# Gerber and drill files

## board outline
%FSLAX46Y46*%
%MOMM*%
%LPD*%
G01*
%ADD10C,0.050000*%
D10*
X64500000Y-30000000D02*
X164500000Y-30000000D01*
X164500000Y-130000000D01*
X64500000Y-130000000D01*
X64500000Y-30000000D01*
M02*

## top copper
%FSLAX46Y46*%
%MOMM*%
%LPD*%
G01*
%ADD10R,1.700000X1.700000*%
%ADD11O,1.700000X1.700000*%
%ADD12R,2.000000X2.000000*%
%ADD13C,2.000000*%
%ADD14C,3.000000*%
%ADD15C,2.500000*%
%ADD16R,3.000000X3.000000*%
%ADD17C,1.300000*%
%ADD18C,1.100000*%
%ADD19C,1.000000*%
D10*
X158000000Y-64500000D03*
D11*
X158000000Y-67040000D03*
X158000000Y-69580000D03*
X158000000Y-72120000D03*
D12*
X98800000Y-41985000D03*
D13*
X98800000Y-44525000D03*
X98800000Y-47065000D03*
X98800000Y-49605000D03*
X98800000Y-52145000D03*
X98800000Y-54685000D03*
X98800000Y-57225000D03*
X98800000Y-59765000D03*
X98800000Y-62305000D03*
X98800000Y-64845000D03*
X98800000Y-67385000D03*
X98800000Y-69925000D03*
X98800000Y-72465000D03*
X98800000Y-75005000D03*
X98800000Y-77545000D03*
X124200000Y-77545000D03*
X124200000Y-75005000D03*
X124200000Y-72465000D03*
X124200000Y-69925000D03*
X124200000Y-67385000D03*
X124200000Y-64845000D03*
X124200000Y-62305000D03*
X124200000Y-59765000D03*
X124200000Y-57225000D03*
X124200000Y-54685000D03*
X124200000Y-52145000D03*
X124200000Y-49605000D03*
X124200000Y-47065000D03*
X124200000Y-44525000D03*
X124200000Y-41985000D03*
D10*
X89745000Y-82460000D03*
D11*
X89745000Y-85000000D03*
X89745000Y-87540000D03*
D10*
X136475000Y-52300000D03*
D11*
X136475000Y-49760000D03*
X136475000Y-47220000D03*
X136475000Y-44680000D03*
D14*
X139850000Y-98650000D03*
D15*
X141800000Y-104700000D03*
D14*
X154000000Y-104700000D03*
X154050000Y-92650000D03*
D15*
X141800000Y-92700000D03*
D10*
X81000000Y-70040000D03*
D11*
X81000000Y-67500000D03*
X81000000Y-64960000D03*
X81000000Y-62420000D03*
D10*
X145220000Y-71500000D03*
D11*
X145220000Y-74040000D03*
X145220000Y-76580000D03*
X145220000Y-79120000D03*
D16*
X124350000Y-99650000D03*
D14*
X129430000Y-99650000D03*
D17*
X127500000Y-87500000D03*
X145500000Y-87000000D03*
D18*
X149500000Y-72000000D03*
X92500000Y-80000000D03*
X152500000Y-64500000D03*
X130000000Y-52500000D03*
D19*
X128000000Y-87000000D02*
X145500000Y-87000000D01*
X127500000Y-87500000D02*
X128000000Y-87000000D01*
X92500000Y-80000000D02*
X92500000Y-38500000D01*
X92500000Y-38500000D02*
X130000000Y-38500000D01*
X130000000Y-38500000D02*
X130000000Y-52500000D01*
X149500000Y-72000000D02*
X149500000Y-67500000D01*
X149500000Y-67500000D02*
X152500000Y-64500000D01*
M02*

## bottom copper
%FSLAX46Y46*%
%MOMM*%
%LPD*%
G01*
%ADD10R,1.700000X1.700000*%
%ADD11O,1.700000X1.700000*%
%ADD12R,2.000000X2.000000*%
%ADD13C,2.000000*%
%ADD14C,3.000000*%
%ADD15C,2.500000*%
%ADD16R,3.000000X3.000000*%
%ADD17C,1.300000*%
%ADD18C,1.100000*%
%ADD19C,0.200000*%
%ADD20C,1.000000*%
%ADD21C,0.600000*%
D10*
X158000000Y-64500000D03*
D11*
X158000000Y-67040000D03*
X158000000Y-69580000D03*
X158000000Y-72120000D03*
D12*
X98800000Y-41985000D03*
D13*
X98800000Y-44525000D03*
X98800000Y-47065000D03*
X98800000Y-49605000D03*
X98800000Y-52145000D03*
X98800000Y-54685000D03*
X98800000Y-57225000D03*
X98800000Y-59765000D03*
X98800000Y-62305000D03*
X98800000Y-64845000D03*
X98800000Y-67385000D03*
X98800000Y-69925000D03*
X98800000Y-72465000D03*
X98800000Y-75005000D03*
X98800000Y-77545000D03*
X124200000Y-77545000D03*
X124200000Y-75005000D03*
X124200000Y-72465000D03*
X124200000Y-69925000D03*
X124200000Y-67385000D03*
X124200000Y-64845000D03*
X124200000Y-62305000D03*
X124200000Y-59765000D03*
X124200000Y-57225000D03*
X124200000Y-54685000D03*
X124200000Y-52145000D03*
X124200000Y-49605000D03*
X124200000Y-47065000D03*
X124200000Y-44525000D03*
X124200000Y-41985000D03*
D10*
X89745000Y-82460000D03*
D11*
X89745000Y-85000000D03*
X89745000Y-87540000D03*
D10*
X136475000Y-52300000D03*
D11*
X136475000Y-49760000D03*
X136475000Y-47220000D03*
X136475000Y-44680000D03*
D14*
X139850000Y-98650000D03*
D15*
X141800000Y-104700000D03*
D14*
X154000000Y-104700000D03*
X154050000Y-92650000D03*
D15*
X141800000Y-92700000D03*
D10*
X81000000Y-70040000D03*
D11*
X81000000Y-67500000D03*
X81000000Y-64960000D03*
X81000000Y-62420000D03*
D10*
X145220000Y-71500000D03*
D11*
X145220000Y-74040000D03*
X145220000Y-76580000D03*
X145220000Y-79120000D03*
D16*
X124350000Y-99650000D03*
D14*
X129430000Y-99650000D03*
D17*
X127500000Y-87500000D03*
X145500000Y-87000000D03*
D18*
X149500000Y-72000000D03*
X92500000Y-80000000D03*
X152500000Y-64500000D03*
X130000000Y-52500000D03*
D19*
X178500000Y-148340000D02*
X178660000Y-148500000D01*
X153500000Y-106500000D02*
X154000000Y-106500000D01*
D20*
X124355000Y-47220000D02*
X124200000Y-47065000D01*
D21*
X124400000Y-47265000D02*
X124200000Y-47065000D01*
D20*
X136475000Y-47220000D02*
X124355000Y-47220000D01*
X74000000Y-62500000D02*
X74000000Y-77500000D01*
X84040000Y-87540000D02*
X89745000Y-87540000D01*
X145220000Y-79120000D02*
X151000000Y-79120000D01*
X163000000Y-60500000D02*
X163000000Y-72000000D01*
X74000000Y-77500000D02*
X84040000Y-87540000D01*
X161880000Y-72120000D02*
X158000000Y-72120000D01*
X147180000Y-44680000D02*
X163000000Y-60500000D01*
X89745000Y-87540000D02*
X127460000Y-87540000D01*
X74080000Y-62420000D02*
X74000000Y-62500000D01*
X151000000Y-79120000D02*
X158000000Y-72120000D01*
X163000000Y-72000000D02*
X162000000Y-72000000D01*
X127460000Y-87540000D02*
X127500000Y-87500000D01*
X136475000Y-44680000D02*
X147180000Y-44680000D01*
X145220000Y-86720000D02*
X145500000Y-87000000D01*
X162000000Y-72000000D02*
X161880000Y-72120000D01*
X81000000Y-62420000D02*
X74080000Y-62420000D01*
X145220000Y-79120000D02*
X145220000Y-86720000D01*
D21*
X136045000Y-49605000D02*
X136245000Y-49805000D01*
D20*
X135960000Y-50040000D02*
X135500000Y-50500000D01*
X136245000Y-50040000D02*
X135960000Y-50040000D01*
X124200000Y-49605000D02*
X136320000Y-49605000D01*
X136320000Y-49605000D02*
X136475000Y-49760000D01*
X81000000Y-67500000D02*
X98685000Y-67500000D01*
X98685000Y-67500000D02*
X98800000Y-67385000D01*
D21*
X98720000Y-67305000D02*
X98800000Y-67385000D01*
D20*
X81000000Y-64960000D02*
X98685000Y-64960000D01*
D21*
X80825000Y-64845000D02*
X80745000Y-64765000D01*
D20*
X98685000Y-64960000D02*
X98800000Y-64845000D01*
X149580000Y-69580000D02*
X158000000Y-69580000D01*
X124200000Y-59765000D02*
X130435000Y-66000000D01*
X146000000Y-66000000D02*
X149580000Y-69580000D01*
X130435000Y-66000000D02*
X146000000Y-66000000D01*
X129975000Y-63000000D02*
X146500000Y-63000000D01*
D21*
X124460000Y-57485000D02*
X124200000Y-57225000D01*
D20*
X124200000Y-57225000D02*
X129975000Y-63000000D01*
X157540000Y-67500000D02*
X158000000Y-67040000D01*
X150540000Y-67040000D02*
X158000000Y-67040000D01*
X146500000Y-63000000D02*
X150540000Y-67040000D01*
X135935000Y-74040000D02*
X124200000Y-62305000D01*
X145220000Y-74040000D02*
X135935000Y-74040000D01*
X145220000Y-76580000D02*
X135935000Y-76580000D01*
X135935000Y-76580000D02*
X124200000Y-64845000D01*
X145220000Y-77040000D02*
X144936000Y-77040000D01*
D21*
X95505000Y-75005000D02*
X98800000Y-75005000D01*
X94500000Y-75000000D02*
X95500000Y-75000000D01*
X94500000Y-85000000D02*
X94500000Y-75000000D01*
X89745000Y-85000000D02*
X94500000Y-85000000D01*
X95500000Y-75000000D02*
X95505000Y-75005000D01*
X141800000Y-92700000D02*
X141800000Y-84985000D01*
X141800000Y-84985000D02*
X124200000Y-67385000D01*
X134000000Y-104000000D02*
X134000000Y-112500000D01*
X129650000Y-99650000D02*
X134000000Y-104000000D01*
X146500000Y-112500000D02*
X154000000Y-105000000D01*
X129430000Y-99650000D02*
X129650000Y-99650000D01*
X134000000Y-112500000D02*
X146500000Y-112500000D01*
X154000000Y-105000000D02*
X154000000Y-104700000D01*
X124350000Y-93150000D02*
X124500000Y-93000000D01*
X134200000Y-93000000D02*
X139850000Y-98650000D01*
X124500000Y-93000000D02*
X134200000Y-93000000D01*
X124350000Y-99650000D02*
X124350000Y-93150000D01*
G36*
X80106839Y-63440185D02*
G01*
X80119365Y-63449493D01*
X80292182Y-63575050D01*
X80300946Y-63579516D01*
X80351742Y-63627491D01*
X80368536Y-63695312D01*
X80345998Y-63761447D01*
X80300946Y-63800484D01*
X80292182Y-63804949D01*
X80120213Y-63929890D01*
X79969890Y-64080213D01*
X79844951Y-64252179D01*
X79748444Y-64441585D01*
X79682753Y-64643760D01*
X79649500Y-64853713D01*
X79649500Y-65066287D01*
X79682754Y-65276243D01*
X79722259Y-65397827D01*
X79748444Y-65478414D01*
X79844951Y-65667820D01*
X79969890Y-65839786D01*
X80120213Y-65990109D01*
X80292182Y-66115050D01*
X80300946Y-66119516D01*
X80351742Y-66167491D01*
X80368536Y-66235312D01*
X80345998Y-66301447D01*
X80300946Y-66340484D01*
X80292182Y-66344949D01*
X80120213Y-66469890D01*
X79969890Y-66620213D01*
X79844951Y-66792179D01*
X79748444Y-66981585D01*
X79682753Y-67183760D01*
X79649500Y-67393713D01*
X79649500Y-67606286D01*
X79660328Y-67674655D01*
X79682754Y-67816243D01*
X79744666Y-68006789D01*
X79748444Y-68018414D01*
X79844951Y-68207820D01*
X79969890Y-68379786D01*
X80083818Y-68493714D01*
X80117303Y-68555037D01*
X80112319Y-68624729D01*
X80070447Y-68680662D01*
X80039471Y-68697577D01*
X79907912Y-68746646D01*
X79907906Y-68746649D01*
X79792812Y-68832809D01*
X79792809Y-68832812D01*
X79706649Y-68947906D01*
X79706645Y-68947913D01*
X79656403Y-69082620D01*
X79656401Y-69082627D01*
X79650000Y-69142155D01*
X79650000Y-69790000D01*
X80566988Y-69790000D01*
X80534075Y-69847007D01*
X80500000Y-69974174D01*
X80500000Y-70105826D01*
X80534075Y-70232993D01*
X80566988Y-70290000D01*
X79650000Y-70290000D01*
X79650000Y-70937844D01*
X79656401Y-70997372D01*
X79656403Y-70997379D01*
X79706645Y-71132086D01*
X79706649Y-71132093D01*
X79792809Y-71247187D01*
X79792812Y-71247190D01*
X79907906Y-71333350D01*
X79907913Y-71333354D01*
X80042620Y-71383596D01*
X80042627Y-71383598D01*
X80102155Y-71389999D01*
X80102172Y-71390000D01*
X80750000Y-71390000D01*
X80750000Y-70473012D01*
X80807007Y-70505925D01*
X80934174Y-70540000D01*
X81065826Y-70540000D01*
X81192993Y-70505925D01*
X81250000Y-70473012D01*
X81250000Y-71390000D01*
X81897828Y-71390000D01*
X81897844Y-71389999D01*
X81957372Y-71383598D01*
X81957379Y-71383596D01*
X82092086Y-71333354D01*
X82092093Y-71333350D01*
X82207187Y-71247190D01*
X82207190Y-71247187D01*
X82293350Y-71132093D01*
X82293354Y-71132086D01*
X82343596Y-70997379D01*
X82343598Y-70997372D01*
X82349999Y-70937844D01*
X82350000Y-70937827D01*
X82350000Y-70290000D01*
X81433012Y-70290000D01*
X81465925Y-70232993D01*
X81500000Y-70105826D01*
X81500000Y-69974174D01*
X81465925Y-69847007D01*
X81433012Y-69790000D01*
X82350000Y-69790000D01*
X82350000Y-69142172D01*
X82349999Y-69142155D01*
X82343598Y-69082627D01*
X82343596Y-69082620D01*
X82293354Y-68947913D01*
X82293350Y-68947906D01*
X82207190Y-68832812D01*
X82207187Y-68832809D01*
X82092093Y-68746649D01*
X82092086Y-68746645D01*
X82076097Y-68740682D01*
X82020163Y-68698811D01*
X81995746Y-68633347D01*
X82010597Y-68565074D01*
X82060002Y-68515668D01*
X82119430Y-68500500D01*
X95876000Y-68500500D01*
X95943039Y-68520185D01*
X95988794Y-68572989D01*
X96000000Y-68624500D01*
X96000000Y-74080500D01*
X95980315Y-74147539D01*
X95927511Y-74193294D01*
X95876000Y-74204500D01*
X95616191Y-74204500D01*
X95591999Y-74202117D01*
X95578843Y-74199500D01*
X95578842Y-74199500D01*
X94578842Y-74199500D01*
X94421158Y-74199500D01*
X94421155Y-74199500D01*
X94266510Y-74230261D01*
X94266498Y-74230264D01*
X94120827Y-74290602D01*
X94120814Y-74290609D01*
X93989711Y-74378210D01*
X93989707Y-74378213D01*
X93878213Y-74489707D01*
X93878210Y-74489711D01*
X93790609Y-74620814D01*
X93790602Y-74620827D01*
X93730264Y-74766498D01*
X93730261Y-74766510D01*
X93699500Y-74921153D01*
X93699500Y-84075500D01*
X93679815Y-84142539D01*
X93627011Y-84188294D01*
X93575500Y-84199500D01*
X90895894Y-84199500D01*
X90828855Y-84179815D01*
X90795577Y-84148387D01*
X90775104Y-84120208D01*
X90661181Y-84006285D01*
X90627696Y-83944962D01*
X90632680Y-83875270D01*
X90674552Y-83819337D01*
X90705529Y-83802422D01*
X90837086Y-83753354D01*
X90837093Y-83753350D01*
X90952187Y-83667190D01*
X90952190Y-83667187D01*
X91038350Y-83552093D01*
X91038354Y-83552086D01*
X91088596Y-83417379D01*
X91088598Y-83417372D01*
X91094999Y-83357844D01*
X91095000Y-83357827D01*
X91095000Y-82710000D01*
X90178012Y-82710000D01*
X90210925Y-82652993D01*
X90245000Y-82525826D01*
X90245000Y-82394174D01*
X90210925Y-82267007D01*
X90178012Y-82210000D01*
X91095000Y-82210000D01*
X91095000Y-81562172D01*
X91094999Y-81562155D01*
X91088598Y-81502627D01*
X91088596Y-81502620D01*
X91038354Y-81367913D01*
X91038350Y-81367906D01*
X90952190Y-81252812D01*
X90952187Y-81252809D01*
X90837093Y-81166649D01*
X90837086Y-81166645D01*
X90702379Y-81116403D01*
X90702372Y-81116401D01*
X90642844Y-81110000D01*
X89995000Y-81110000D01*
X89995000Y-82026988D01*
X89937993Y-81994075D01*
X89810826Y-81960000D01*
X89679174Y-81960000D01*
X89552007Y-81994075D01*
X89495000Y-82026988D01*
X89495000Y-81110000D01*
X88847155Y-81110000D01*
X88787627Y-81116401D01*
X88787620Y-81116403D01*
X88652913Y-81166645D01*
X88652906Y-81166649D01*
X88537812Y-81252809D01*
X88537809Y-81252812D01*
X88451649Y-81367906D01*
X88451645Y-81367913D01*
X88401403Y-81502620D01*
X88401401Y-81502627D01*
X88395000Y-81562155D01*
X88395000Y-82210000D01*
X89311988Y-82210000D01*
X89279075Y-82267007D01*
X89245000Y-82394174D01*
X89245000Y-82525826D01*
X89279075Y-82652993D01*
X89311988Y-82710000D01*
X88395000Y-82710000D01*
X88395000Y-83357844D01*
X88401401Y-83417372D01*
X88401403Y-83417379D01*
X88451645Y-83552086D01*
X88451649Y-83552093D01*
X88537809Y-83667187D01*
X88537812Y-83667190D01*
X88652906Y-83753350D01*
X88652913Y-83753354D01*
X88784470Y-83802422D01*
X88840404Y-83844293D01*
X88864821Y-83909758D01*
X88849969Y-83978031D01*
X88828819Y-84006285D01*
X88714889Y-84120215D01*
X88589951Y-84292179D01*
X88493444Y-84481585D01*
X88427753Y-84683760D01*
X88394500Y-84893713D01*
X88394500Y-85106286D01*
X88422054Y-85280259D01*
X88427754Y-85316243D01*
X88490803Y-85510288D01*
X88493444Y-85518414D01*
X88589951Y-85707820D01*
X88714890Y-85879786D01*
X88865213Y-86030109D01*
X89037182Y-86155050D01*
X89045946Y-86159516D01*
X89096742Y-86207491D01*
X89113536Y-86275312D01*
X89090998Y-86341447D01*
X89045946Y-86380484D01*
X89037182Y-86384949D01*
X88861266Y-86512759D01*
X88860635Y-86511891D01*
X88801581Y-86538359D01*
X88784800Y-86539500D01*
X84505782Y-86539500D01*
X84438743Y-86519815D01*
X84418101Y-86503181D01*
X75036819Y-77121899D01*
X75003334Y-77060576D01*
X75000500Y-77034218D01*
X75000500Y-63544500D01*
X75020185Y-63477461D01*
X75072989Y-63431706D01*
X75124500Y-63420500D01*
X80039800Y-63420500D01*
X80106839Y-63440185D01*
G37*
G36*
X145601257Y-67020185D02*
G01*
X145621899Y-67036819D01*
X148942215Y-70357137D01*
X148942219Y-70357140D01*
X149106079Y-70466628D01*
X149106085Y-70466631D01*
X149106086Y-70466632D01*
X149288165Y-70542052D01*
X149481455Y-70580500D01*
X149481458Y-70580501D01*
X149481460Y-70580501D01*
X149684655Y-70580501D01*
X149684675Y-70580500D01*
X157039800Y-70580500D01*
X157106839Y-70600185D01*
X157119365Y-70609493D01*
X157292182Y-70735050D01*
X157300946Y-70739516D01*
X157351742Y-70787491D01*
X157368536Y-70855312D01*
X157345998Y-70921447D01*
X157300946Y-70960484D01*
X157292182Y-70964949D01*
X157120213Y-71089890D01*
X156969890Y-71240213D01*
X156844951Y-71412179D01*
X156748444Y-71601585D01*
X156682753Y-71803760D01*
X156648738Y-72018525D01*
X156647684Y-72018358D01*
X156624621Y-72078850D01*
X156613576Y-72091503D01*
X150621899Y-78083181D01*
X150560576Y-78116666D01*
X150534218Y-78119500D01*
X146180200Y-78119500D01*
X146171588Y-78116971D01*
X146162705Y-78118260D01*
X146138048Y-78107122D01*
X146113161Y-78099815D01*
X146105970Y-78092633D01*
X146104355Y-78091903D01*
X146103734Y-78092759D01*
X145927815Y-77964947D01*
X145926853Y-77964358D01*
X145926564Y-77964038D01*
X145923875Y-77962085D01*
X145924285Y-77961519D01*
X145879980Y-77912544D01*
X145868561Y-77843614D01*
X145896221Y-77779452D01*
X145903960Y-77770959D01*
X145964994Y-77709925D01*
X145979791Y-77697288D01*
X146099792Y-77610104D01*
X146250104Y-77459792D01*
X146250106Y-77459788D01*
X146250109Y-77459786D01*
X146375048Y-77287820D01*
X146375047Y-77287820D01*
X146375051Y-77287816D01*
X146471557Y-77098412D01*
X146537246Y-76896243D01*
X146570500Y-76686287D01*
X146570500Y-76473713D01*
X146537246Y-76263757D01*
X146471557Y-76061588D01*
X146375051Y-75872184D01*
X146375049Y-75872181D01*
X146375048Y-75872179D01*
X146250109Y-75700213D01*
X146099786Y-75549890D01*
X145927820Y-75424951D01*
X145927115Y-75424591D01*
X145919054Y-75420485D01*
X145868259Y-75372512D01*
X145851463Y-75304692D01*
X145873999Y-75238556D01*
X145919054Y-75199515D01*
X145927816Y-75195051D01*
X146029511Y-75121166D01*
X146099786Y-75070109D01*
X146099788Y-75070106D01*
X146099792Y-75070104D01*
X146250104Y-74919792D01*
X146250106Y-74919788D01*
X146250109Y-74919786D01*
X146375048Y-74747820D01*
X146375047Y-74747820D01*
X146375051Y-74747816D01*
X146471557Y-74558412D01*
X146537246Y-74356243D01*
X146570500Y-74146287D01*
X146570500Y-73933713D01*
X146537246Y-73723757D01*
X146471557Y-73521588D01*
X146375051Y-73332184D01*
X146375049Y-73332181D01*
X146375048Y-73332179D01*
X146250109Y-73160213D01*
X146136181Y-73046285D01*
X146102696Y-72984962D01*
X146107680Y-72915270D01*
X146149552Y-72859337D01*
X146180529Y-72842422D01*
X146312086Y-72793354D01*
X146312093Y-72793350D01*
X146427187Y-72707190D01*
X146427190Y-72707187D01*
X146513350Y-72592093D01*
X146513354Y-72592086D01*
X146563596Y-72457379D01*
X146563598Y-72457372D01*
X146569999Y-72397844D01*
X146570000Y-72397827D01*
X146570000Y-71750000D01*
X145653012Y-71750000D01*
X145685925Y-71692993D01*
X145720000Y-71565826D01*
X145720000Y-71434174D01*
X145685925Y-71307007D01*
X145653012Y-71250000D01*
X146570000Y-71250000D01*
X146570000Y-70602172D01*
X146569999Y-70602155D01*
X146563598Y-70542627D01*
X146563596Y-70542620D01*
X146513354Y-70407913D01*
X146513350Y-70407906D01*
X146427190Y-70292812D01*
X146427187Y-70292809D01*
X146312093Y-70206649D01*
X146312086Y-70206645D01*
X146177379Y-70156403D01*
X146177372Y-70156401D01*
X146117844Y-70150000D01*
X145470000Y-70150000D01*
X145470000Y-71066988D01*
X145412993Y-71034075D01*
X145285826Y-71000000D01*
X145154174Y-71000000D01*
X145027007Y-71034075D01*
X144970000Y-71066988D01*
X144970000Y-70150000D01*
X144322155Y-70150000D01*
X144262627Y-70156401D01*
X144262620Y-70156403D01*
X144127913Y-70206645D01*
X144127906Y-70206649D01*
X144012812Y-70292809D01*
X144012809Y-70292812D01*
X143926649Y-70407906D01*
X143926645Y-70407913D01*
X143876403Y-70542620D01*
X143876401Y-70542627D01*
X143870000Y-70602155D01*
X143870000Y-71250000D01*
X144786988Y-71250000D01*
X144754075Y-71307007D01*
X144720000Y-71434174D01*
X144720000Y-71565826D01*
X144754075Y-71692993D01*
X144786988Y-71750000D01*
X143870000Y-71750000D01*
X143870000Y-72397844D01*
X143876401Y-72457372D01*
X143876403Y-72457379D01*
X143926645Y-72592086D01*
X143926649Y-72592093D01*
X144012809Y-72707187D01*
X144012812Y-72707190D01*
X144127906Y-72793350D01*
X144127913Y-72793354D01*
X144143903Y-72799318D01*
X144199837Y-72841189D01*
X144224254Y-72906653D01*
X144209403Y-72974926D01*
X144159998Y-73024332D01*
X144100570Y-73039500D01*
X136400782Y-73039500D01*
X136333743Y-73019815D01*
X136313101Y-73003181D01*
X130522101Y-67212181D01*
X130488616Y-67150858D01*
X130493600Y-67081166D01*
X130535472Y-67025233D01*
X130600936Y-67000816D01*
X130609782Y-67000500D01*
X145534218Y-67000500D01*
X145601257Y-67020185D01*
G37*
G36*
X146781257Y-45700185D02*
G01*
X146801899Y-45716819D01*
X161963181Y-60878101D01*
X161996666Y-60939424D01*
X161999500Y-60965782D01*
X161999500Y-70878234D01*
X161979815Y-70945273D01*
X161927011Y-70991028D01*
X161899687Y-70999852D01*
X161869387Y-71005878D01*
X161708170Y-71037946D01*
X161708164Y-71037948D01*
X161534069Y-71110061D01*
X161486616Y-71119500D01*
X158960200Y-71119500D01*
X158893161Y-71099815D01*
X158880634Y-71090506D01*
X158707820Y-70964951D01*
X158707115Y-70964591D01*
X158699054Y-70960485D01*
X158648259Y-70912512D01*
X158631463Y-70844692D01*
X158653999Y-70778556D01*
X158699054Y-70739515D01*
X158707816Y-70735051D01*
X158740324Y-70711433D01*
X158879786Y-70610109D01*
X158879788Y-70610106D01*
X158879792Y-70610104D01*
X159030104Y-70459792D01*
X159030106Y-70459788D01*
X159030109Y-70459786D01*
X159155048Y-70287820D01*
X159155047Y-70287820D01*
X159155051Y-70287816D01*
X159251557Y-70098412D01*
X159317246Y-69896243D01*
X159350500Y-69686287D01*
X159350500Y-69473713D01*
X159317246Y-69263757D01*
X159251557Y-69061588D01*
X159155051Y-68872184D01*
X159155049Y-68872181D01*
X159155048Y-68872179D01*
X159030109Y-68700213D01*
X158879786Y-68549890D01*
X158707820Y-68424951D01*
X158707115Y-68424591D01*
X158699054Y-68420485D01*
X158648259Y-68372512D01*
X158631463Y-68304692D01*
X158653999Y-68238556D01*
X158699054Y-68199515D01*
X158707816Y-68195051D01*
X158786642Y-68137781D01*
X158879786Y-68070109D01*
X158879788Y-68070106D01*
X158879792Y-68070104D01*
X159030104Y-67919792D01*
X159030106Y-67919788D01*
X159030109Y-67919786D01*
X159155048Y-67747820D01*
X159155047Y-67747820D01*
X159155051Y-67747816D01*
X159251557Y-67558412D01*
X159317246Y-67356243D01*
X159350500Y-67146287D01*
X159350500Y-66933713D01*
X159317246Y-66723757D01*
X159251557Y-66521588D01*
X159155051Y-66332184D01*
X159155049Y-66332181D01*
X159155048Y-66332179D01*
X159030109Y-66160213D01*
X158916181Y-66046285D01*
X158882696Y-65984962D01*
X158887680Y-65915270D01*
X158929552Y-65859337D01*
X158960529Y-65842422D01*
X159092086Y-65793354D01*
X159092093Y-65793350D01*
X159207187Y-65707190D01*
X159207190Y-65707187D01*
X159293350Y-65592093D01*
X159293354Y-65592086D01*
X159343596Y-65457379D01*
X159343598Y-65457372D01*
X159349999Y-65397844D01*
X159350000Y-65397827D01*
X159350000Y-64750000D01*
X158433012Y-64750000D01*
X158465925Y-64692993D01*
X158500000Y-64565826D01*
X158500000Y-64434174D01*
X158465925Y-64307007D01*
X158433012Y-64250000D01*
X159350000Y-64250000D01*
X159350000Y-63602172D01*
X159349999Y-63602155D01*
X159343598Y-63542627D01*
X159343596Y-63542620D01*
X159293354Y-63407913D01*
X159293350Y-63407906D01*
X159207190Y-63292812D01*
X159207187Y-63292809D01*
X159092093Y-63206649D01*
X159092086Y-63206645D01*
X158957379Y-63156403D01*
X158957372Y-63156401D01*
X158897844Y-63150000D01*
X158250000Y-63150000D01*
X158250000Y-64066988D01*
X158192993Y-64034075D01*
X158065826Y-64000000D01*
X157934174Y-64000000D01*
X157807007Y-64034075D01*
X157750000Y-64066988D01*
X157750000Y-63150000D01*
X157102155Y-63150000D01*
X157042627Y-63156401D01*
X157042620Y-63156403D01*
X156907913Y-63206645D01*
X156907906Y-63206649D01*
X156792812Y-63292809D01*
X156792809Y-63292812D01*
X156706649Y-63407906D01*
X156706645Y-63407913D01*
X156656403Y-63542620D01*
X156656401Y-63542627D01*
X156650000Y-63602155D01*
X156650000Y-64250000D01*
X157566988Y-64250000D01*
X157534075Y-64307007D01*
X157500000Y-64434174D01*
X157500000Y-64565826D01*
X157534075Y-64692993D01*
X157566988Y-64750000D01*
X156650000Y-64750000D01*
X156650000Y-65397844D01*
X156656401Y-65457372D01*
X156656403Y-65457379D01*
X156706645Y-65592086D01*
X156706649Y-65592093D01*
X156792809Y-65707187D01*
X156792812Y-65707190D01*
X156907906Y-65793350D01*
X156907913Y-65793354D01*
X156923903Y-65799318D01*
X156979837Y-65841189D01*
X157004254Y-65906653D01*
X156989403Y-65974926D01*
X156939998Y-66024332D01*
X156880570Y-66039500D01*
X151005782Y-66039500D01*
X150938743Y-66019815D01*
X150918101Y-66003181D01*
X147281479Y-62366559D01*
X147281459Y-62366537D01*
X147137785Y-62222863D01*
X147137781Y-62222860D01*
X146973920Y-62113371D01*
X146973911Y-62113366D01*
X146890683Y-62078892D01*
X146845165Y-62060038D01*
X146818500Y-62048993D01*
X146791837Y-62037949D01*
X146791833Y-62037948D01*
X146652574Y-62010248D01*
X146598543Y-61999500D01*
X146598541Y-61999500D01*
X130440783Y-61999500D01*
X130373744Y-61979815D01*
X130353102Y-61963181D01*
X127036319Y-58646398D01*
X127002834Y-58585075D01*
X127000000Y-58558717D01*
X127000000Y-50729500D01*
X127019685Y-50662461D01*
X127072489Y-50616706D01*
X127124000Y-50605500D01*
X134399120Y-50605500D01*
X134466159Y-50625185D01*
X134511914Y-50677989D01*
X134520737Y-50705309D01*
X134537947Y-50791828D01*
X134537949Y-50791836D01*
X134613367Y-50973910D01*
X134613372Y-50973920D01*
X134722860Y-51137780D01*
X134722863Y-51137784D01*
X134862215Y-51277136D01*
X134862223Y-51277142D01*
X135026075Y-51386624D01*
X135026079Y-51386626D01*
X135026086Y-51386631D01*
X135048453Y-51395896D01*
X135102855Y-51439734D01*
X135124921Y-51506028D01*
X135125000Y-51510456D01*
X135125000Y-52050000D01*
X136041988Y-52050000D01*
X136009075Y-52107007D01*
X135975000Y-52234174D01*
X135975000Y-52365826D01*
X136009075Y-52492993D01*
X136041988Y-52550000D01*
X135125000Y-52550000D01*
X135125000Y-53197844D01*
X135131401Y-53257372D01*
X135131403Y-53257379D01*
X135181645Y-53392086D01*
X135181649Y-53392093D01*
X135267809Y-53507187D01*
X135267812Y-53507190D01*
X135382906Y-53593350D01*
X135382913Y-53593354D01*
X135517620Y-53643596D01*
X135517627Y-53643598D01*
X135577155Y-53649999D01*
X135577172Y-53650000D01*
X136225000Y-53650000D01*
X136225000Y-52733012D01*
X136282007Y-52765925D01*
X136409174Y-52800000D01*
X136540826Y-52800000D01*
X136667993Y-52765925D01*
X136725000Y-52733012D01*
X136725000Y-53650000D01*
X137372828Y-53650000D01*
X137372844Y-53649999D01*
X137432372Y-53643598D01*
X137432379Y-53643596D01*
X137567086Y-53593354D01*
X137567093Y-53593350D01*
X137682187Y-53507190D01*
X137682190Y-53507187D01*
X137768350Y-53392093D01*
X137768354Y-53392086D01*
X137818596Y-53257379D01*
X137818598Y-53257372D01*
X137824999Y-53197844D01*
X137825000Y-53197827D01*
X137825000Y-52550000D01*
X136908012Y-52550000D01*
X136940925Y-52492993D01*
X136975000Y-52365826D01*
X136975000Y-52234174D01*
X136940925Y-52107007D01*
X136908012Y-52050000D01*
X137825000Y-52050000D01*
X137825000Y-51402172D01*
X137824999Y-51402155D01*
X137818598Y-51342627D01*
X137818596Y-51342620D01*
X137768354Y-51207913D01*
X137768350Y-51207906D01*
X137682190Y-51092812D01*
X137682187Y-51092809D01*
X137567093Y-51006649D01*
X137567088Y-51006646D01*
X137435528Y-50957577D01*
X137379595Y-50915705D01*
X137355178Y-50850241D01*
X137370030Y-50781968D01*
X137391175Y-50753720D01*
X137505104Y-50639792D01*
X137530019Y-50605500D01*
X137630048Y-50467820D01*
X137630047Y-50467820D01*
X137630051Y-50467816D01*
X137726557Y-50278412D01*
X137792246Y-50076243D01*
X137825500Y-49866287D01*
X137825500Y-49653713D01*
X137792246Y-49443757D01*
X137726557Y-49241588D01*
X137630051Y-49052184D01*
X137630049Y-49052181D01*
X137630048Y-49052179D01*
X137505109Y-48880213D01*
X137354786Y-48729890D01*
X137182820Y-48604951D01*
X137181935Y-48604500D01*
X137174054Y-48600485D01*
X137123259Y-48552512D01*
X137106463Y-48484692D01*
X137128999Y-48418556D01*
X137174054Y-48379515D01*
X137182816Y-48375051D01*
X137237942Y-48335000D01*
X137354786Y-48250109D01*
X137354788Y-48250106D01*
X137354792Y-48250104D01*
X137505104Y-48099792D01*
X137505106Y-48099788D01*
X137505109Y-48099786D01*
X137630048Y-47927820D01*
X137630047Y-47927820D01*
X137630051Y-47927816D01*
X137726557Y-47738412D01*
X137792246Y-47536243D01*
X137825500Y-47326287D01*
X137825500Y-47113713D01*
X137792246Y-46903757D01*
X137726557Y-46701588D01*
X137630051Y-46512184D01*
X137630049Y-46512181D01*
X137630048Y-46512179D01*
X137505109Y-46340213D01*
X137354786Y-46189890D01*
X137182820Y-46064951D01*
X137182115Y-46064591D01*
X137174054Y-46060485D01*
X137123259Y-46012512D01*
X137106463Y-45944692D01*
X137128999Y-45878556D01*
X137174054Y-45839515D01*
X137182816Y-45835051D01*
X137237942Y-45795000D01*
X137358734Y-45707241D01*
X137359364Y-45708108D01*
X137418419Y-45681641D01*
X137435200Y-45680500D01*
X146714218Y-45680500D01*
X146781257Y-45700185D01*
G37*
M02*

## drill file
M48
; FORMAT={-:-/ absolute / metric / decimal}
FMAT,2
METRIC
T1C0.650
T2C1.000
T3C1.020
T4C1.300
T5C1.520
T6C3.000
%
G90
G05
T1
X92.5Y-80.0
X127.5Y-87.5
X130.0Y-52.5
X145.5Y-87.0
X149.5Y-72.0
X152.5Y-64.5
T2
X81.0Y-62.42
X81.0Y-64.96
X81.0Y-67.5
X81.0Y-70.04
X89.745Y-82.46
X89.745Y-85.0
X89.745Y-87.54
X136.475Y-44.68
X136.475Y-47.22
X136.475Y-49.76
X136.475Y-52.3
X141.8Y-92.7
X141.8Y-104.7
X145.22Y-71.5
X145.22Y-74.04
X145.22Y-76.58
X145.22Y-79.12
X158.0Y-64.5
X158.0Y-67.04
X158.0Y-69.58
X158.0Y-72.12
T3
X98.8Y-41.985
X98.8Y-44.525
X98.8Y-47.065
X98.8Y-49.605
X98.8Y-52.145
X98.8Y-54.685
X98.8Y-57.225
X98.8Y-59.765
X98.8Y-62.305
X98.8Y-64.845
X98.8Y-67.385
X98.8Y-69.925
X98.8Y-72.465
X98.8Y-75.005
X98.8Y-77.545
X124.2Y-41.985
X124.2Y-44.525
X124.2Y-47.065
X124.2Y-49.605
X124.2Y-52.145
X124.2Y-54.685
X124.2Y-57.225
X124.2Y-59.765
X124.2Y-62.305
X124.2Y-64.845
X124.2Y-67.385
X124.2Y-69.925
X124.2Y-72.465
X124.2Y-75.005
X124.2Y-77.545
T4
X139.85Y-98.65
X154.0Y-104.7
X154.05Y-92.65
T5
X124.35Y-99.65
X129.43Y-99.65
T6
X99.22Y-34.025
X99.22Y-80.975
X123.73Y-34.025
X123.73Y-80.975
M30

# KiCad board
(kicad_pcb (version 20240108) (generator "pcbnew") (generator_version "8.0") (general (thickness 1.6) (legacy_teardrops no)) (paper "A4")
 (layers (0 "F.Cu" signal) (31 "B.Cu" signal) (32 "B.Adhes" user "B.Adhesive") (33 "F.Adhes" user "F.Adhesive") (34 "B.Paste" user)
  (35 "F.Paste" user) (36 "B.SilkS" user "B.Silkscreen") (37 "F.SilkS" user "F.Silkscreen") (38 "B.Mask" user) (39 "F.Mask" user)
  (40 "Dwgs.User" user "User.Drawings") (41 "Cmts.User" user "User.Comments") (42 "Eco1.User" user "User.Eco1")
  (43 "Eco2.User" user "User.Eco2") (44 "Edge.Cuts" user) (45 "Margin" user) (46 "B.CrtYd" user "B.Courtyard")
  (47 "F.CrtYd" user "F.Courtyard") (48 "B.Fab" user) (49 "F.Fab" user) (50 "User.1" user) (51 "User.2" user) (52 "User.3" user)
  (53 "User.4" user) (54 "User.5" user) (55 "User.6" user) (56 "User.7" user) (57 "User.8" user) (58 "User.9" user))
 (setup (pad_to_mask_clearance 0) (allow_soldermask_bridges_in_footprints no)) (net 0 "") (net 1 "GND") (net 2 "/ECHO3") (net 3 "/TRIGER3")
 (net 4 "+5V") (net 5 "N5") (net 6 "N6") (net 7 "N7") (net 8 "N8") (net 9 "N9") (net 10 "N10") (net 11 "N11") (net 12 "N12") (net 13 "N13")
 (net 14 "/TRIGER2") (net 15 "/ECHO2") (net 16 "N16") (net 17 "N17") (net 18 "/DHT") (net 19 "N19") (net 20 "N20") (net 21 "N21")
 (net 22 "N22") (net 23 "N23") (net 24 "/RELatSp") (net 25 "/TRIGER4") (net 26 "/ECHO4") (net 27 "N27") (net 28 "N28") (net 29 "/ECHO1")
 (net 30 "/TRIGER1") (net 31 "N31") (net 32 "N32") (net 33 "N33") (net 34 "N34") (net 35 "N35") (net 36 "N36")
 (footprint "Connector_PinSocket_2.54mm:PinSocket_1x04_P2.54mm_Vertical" (layer "F.Cu") (at 158 64.5)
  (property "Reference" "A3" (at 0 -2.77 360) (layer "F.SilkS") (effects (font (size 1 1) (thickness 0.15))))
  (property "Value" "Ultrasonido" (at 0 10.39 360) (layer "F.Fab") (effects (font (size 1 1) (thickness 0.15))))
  (pad "1" thru_hole rect (at 0 0) (size 1.7 1.7) (drill 1) (layers "*.Cu" "*.Mask") (remove_unused_layers no) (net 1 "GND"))
  (pad "2" thru_hole oval (at 0 2.54) (size 1.7 1.7) (drill 1) (layers "*.Cu" "*.Mask") (remove_unused_layers no) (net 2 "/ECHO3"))
  (pad "3" thru_hole oval (at 0 5.08) (size 1.7 1.7) (drill 1) (layers "*.Cu" "*.Mask") (remove_unused_layers no) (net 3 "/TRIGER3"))
  (pad "4" thru_hole oval (at 0 7.62) (size 1.7 1.7) (drill 1) (layers "*.Cu" "*.Mask") (remove_unused_layers no) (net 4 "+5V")))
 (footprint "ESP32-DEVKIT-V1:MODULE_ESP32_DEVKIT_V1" (layer "F.Cu") (at 111.5 57.5)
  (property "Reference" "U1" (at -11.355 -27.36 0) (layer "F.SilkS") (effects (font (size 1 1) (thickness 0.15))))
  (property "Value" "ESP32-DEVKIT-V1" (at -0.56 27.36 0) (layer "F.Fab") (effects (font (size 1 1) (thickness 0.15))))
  (pad "" np_thru_hole circle (at -12.28 -23.475) (size 3 3) (drill 3) (layers "*.Cu" "*.Mask"))
  (pad "" np_thru_hole circle (at -12.28 23.475) (size 3 3) (drill 3) (layers "*.Cu" "*.Mask"))
  (pad "" np_thru_hole circle (at 12.23 -23.475) (size 3 3) (drill 3) (layers "*.Cu" "*.Mask"))
  (pad "" np_thru_hole circle (at 12.23 23.475) (size 3 3) (drill 3) (layers "*.Cu" "*.Mask"))
  (pad "1" thru_hole rect (at -12.7 -15.515) (size 2 2) (drill 1.02) (layers "*.Cu" "*.Mask") (remove_unused_layers no) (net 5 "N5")
   (solder_mask_margin 0.102))
  (pad "2" thru_hole circle (at -12.7 -12.975) (size 2 2) (drill 1.02) (layers "*.Cu" "*.Mask") (remove_unused_layers no) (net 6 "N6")
   (solder_mask_margin 0.102))
  (pad "3" thru_hole circle (at -12.7 -10.435) (size 2 2) (drill 1.02) (layers "*.Cu" "*.Mask") (remove_unused_layers no) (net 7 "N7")
   (solder_mask_margin 0.102))
  (pad "4" thru_hole circle (at -12.7 -7.895) (size 2 2) (drill 1.02) (layers "*.Cu" "*.Mask") (remove_unused_layers no) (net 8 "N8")
   (solder_mask_margin 0.102))
  (pad "5" thru_hole circle (at -12.7 -5.355) (size 2 2) (drill 1.02) (layers "*.Cu" "*.Mask") (remove_unused_layers no) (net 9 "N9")
   (solder_mask_margin 0.102))
  (pad "6" thru_hole circle (at -12.7 -2.815) (size 2 2) (drill 1.02) (layers "*.Cu" "*.Mask") (remove_unused_layers no) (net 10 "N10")
   (solder_mask_margin 0.102))
  (pad "7" thru_hole circle (at -12.7 -0.275) (size 2 2) (drill 1.02) (layers "*.Cu" "*.Mask") (remove_unused_layers no) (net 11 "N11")
   (solder_mask_margin 0.102))
  (pad "8" thru_hole circle (at -12.7 2.265) (size 2 2) (drill 1.02) (layers "*.Cu" "*.Mask") (remove_unused_layers no) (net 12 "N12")
   (solder_mask_margin 0.102))
  (pad "9" thru_hole circle (at -12.7 4.805) (size 2 2) (drill 1.02) (layers "*.Cu" "*.Mask") (remove_unused_layers no) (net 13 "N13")
   (solder_mask_margin 0.102))
  (pad "10" thru_hole circle (at -12.7 7.345) (size 2 2) (drill 1.02) (layers "*.Cu" "*.Mask") (remove_unused_layers no) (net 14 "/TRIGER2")
   (solder_mask_margin 0.102))
  (pad "11" thru_hole circle (at -12.7 9.885) (size 2 2) (drill 1.02) (layers "*.Cu" "*.Mask") (remove_unused_layers no) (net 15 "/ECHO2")
   (solder_mask_margin 0.102))
  (pad "12" thru_hole circle (at -12.7 12.425) (size 2 2) (drill 1.02) (layers "*.Cu" "*.Mask") (remove_unused_layers no) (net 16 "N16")
   (solder_mask_margin 0.102))
  (pad "13" thru_hole circle (at -12.7 14.965) (size 2 2) (drill 1.02) (layers "*.Cu" "*.Mask") (remove_unused_layers no) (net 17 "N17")
   (solder_mask_margin 0.102))
  (pad "14" thru_hole circle (at -12.7 17.505) (size 2 2) (drill 1.02) (layers "*.Cu" "*.Mask") (remove_unused_layers no) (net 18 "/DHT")
   (solder_mask_margin 0.102))
  (pad "15" thru_hole circle (at -12.7 20.045) (size 2 2) (drill 1.02) (layers "*.Cu" "*.Mask") (remove_unused_layers no) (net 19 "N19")
   (solder_mask_margin 0.102))
  (pad "16" thru_hole circle (at 12.7 20.045) (size 2 2) (drill 1.02) (layers "*.Cu" "*.Mask") (remove_unused_layers no) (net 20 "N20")
   (solder_mask_margin 0.102))
  (pad "17" thru_hole circle (at 12.7 17.505) (size 2 2) (drill 1.02) (layers "*.Cu" "*.Mask") (remove_unused_layers no) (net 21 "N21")
   (solder_mask_margin 0.102))
  (pad "18" thru_hole circle (at 12.7 14.965) (size 2 2) (drill 1.02) (layers "*.Cu" "*.Mask") (remove_unused_layers no) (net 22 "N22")
   (solder_mask_margin 0.102))
  (pad "19" thru_hole circle (at 12.7 12.425) (size 2 2) (drill 1.02) (layers "*.Cu" "*.Mask") (remove_unused_layers no) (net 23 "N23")
   (solder_mask_margin 0.102))
  (pad "20" thru_hole circle (at 12.7 9.885) (size 2 2) (drill 1.02) (layers "*.Cu" "*.Mask") (remove_unused_layers no) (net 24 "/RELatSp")
   (solder_mask_margin 0.102))
  (pad "21" thru_hole circle (at 12.7 7.345) (size 2 2) (drill 1.02) (layers "*.Cu" "*.Mask") (remove_unused_layers no) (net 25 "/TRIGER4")
   (solder_mask_margin 0.102))
  (pad "22" thru_hole circle (at 12.7 4.805) (size 2 2) (drill 1.02) (layers "*.Cu" "*.Mask") (remove_unused_layers no) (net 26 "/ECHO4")
   (solder_mask_margin 0.102))
  (pad "23" thru_hole circle (at 12.7 2.265) (size 2 2) (drill 1.02) (layers "*.Cu" "*.Mask") (remove_unused_layers no) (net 3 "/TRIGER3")
   (solder_mask_margin 0.102))
  (pad "24" thru_hole circle (at 12.7 -0.275) (size 2 2) (drill 1.02) (layers "*.Cu" "*.Mask") (remove_unused_layers no) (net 2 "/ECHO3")
   (solder_mask_margin 0.102))
  (pad "25" thru_hole circle (at 12.7 -2.815) (size 2 2) (drill 1.02) (layers "*.Cu" "*.Mask") (remove_unused_layers no) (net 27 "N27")
   (solder_mask_margin 0.102))
  (pad "26" thru_hole circle (at 12.7 -5.355) (size 2 2) (drill 1.02) (layers "*.Cu" "*.Mask") (remove_unused_layers no) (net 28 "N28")
   (solder_mask_margin 0.102))
  (pad "27" thru_hole circle (at 12.7 -7.895) (size 2 2) (drill 1.02) (layers "*.Cu" "*.Mask") (remove_unused_layers no) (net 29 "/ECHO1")
   (solder_mask_margin 0.102))
  (pad "28" thru_hole circle (at 12.7 -10.435) (size 2 2) (drill 1.02) (layers "*.Cu" "*.Mask") (remove_unused_layers no)
   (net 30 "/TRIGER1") (solder_mask_margin 0.102))
  (pad "29" thru_hole circle (at 12.7 -12.975) (size 2 2) (drill 1.02) (layers "*.Cu" "*.Mask") (remove_unused_layers no) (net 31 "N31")
   (solder_mask_margin 0.102))
  (pad "30" thru_hole circle (at 12.7 -15.515) (size 2 2) (drill 1.02) (layers "*.Cu" "*.Mask") (remove_unused_layers no) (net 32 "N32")
   (solder_mask_margin 0.102))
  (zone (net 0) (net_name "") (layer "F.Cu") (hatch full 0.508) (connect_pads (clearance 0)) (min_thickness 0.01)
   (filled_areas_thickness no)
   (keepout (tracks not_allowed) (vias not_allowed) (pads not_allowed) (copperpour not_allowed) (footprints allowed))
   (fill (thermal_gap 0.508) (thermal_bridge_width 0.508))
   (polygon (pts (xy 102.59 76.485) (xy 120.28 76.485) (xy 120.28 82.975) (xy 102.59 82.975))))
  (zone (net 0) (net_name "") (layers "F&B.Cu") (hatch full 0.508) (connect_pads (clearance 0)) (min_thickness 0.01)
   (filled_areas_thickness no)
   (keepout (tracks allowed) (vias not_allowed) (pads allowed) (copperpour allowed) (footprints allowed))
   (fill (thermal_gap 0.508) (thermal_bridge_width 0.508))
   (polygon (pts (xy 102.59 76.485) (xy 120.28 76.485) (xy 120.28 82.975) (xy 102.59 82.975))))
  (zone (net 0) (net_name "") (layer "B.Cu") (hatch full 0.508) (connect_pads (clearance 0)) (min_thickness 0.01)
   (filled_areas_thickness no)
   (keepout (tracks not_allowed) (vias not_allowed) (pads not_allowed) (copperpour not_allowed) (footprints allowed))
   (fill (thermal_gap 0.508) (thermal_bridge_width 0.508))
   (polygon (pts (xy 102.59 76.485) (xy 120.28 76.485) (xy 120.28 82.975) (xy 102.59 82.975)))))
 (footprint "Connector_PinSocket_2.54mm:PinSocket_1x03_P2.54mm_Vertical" (layer "F.Cu") (at 89.745 82.46)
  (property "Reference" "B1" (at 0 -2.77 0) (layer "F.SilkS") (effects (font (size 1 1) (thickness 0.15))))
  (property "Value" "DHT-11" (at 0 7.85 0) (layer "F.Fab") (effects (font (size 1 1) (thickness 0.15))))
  (pad "1" thru_hole rect (at 0 0) (size 1.7 1.7) (drill 1) (layers "*.Cu" "*.Mask") (remove_unused_layers no) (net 1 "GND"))
  (pad "2" thru_hole oval (at 0 2.54) (size 1.7 1.7) (drill 1) (layers "*.Cu" "*.Mask") (remove_unused_layers no) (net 18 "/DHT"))
  (pad "3" thru_hole oval (at 0 5.08) (size 1.7 1.7) (drill 1) (layers "*.Cu" "*.Mask") (remove_unused_layers no) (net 4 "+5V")))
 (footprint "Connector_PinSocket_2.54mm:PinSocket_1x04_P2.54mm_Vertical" (layer "F.Cu") (at 136.475 52.3 180)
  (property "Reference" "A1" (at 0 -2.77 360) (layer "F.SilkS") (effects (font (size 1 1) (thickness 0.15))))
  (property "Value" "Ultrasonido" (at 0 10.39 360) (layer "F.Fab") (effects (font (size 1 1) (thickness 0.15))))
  (pad "1" thru_hole rect (at 0 0 180) (size 1.7 1.7) (drill 1) (layers "*.Cu" "*.Mask") (remove_unused_layers no) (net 1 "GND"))
  (pad "2" thru_hole oval (at 0 2.54 180) (size 1.7 1.7) (drill 1) (layers "*.Cu" "*.Mask") (remove_unused_layers no) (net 29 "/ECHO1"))
  (pad "3" thru_hole oval (at 0 5.08 180) (size 1.7 1.7) (drill 1) (layers "*.Cu" "*.Mask") (remove_unused_layers no) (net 30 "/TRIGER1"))
  (pad "4" thru_hole oval (at 0 7.62 180) (size 1.7 1.7) (drill 1) (layers "*.Cu" "*.Mask") (remove_unused_layers no) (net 4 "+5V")))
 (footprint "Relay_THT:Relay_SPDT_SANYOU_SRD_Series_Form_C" (layer "F.Cu") (at 139.85 98.65)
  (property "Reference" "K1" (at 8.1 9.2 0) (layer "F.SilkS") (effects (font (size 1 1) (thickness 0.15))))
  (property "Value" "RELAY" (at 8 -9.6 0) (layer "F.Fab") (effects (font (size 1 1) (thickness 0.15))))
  (pad "1" thru_hole circle (at 0 0 90) (size 3 3) (drill 1.3) (layers "*.Cu" "*.Mask") (remove_unused_layers no) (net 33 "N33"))
  (pad "2" thru_hole circle (at 1.95 6.05 90) (size 2.5 2.5) (drill 1) (layers "*.Cu" "*.Mask") (remove_unused_layers no) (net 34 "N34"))
  (pad "3" thru_hole circle (at 14.15 6.05 90) (size 3 3) (drill 1.3) (layers "*.Cu" "*.Mask") (remove_unused_layers no) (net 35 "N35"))
  (pad "4" thru_hole circle (at 14.2 -6 90) (size 3 3) (drill 1.3) (layers "*.Cu" "*.Mask") (remove_unused_layers no) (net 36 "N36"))
  (pad "5" thru_hole circle (at 1.95 -5.95 90) (size 2.5 2.5) (drill 1) (layers "*.Cu" "*.Mask") (remove_unused_layers no)
   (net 24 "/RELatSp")))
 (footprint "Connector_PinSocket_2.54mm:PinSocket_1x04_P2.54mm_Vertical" (layer "F.Cu") (at 81 70.04 180)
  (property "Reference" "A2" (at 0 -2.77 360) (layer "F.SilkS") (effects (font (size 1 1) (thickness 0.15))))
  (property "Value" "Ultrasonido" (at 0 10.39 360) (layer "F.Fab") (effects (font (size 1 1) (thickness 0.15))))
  (pad "1" thru_hole rect (at 0 0 180) (size 1.7 1.7) (drill 1) (layers "*.Cu" "*.Mask") (remove_unused_layers no) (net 1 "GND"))
  (pad "2" thru_hole oval (at 0 2.54 180) (size 1.7 1.7) (drill 1) (layers "*.Cu" "*.Mask") (remove_unused_layers no) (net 15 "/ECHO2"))
  (pad "3" thru_hole oval (at 0 5.08 180) (size 1.7 1.7) (drill 1) (layers "*.Cu" "*.Mask") (remove_unused_layers no) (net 14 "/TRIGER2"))
  (pad "4" thru_hole oval (at 0 7.62 180) (size 1.7 1.7) (drill 1) (layers "*.Cu" "*.Mask") (remove_unused_layers no) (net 4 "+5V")))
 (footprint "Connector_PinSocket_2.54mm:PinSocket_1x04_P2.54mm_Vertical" (layer "F.Cu") (at 145.22 71.5)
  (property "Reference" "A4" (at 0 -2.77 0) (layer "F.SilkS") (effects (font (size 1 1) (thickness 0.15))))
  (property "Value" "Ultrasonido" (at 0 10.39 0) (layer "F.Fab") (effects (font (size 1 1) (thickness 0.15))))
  (pad "1" thru_hole rect (at 0 0) (size 1.7 1.7) (drill 1) (layers "*.Cu" "*.Mask") (remove_unused_layers no) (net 1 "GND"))
  (pad "2" thru_hole oval (at 0 2.54) (size 1.7 1.7) (drill 1) (layers "*.Cu" "*.Mask") (remove_unused_layers no) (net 26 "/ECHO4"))
  (pad "3" thru_hole oval (at 0 5.08) (size 1.7 1.7) (drill 1) (layers "*.Cu" "*.Mask") (remove_unused_layers no) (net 25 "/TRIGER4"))
  (pad "4" thru_hole oval (at 0 7.62) (size 1.7 1.7) (drill 1) (layers "*.Cu" "*.Mask") (remove_unused_layers no) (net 4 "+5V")))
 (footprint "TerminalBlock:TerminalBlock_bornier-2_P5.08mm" (layer "F.Cu") (at 124.35 99.65)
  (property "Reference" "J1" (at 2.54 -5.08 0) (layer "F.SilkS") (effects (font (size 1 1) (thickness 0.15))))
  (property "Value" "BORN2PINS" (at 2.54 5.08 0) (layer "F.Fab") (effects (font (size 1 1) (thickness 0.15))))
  (pad "1" thru_hole rect (at 0 0) (size 3 3) (drill 1.52) (layers "*.Cu" "*.Mask") (remove_unused_layers no) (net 33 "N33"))
  (pad "2" thru_hole circle (at 5.08 0) (size 3 3) (drill 1.52) (layers "*.Cu" "*.Mask") (remove_unused_layers no) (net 35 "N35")))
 (gr_rect (start 64.5 30) (end 164.5 130) (stroke (width 0.05) (type default)) (fill none) (layer "Edge.Cuts"))
 (segment (start 178.5 148.34) (end 178.66 148.5) (width 0.2) (layer "B.Cu") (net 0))
 (segment (start 153.5 106.5) (end 154 106.5) (width 0.2) (layer "B.Cu") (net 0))
 (segment (start 124.355 47.22) (end 124.2 47.065) (width 1) (layer "B.Cu") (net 30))
 (segment (start 124.4 47.265) (end 124.2 47.065) (width 0.6) (layer "B.Cu") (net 30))
 (segment (start 136.475 47.22) (end 124.355 47.22) (width 1) (layer "B.Cu") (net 30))
 (segment (start 128 87) (end 145.5 87) (width 1) (layer "F.Cu") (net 4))
 (segment (start 127.5 87.5) (end 128 87) (width 1) (layer "F.Cu") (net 4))
 (via (at 127.5 87.5) (size 1.3) (drill 0.65) (layers "F.Cu" "B.Cu") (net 4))
 (via (at 145.5 87) (size 1.3) (drill 0.65) (layers "F.Cu" "B.Cu") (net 4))
 (segment (start 74 62.5) (end 74 77.5) (width 1) (layer "B.Cu") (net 4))
 (segment (start 84.04 87.54) (end 89.745 87.54) (width 1) (layer "B.Cu") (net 4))
 (segment (start 145.22 79.12) (end 151 79.12) (width 1) (layer "B.Cu") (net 4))
 (segment (start 163 60.5) (end 163 72) (width 1) (layer "B.Cu") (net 4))
 (segment (start 74 77.5) (end 84.04 87.54) (width 1) (layer "B.Cu") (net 4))
 (segment (start 161.88 72.12) (end 158 72.12) (width 1) (layer "B.Cu") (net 4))
 (segment (start 147.18 44.68) (end 163 60.5) (width 1) (layer "B.Cu") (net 4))
 (segment (start 89.745 87.54) (end 127.46 87.54) (width 1) (layer "B.Cu") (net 4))
 (segment (start 74.08 62.42) (end 74 62.5) (width 1) (layer "B.Cu") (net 4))
 (segment (start 151 79.12) (end 158 72.12) (width 1) (layer "B.Cu") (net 4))
 (segment (start 163 72) (end 162 72) (width 1) (layer "B.Cu") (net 4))
 (segment (start 127.46 87.54) (end 127.5 87.5) (width 1) (layer "B.Cu") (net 4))
 (segment (start 136.475 44.68) (end 147.18 44.68) (width 1) (layer "B.Cu") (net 4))
 (segment (start 145.22 86.72) (end 145.5 87) (width 1) (layer "B.Cu") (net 4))
 (segment (start 162 72) (end 161.88 72.12) (width 1) (layer "B.Cu") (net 4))
 (segment (start 81 62.42) (end 74.08 62.42) (width 1) (layer "B.Cu") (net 4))
 (segment (start 145.22 79.12) (end 145.22 86.72) (width 1) (layer "B.Cu") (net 4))
 (segment (start 92.5 80) (end 92.5 38.5) (width 1) (layer "F.Cu") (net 1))
 (segment (start 92.5 38.5) (end 130 38.5) (width 1) (layer "F.Cu") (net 1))
 (segment (start 130 38.5) (end 130 52.5) (width 1) (layer "F.Cu") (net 1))
 (segment (start 149.5 72) (end 149.5 67.5) (width 1) (layer "F.Cu") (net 1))
 (segment (start 149.5 67.5) (end 152.5 64.5) (width 1) (layer "F.Cu") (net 1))
 (via (at 149.5 72) (size 1.1) (drill 0.65) (layers "F.Cu" "B.Cu") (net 1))
 (via (at 92.5 80) (size 1.1) (drill 0.65) (layers "F.Cu" "B.Cu") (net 1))
 (via (at 152.5 64.5) (size 1.1) (drill 0.65) (layers "F.Cu" "B.Cu") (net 1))
 (via (at 130 52.5) (size 1.1) (drill 0.65) (layers "F.Cu" "B.Cu") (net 1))
 (segment (start 136.045 49.605) (end 136.245 49.805) (width 0.6) (layer "B.Cu") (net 29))
 (segment (start 135.96 50.04) (end 135.5 50.5) (width 1) (layer "B.Cu") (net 29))
 (segment (start 136.245 50.04) (end 135.96 50.04) (width 1) (layer "B.Cu") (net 29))
 (segment (start 124.2 49.605) (end 136.32 49.605) (width 1) (layer "B.Cu") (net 29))
 (segment (start 136.32 49.605) (end 136.475 49.76) (width 1) (layer "B.Cu") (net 29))
 (segment (start 81 67.5) (end 98.685 67.5) (width 1) (layer "B.Cu") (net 15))
 (segment (start 98.685 67.5) (end 98.8 67.385) (width 1) (layer "B.Cu") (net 15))
 (segment (start 98.72 67.305) (end 98.8 67.385) (width 0.6) (layer "B.Cu") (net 15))
 (segment (start 81 64.96) (end 98.685 64.96) (width 1) (layer "B.Cu") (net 14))
 (segment (start 80.825 64.845) (end 80.745 64.765) (width 0.6) (layer "B.Cu") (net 14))
 (segment (start 98.685 64.96) (end 98.8 64.845) (width 1) (layer "B.Cu") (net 14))
 (segment (start 149.58 69.58) (end 158 69.58) (width 1) (layer "B.Cu") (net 3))
 (segment (start 124.2 59.765) (end 130.435 66) (width 1) (layer "B.Cu") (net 3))
 (segment (start 146 66) (end 149.58 69.58) (width 1) (layer "B.Cu") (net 3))
 (segment (start 130.435 66) (end 146 66) (width 1) (layer "B.Cu") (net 3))
 (segment (start 129.975 63) (end 146.5 63) (width 1) (layer "B.Cu") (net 2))
 (segment (start 124.46 57.485) (end 124.2 57.225) (width 0.6) (layer "B.Cu") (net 2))
 (segment (start 124.2 57.225) (end 129.975 63) (width 1) (layer "B.Cu") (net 2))
 (segment (start 157.54 67.5) (end 158 67.04) (width 1) (layer "B.Cu") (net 2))
 (segment (start 150.54 67.04) (end 158 67.04) (width 1) (layer "B.Cu") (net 2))
 (segment (start 146.5 63) (end 150.54 67.04) (width 1) (layer "B.Cu") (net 2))
 (segment (start 135.935 74.04) (end 124.2 62.305) (width 1) (layer "B.Cu") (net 26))
 (segment (start 145.22 74.04) (end 135.935 74.04) (width 1) (layer "B.Cu") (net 26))
 (segment (start 145.22 76.58) (end 135.935 76.58) (width 1) (layer "B.Cu") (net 25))
 (segment (start 135.935 76.58) (end 124.2 64.845) (width 1) (layer "B.Cu") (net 25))
 (segment (start 145.22 77.04) (end 144.936 77.04) (width 1) (layer "B.Cu") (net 25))
 (segment (start 95.505 75.005) (end 98.8 75.005) (width 0.6) (layer "B.Cu") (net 18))
 (segment (start 94.5 75) (end 95.5 75) (width 0.6) (layer "B.Cu") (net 18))
 (segment (start 94.5 85) (end 94.5 75) (width 0.6) (layer "B.Cu") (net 18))
 (segment (start 89.745 85) (end 94.5 85) (width 0.6) (layer "B.Cu") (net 18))
 (segment (start 95.5 75) (end 95.505 75.005) (width 0.6) (layer "B.Cu") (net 18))
 (segment (start 141.8 92.7) (end 141.8 84.985) (width 0.6) (layer "B.Cu") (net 24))
 (segment (start 141.8 84.985) (end 124.2 67.385) (width 0.6) (layer "B.Cu") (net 24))
 (segment (start 134 104) (end 134 112.5) (width 0.6) (layer "B.Cu") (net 35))
 (segment (start 129.65 99.65) (end 134 104) (width 0.6) (layer "B.Cu") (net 35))
 (segment (start 146.5 112.5) (end 154 105) (width 0.6) (layer "B.Cu") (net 35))
 (segment (start 129.43 99.65) (end 129.65 99.65) (width 0.6) (layer "B.Cu") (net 35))
 (segment (start 134 112.5) (end 146.5 112.5) (width 0.6) (layer "B.Cu") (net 35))
 (segment (start 154 105) (end 154 104.7) (width 0.6) (layer "B.Cu") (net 35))
 (segment (start 124.35 93.15) (end 124.5 93) (width 0.6) (layer "B.Cu") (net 33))
 (segment (start 134.2 93) (end 139.85 98.65) (width 0.6) (layer "B.Cu") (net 33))
 (segment (start 124.5 93) (end 134.2 93) (width 0.6) (layer "B.Cu") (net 33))
 (segment (start 124.35 99.65) (end 124.35 93.15) (width 0.6) (layer "B.Cu") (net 33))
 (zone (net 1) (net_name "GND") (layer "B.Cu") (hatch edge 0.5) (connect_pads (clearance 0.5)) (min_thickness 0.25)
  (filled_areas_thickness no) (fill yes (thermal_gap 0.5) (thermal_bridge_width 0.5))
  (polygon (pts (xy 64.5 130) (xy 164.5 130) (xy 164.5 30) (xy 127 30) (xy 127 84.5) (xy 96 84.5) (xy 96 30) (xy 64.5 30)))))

